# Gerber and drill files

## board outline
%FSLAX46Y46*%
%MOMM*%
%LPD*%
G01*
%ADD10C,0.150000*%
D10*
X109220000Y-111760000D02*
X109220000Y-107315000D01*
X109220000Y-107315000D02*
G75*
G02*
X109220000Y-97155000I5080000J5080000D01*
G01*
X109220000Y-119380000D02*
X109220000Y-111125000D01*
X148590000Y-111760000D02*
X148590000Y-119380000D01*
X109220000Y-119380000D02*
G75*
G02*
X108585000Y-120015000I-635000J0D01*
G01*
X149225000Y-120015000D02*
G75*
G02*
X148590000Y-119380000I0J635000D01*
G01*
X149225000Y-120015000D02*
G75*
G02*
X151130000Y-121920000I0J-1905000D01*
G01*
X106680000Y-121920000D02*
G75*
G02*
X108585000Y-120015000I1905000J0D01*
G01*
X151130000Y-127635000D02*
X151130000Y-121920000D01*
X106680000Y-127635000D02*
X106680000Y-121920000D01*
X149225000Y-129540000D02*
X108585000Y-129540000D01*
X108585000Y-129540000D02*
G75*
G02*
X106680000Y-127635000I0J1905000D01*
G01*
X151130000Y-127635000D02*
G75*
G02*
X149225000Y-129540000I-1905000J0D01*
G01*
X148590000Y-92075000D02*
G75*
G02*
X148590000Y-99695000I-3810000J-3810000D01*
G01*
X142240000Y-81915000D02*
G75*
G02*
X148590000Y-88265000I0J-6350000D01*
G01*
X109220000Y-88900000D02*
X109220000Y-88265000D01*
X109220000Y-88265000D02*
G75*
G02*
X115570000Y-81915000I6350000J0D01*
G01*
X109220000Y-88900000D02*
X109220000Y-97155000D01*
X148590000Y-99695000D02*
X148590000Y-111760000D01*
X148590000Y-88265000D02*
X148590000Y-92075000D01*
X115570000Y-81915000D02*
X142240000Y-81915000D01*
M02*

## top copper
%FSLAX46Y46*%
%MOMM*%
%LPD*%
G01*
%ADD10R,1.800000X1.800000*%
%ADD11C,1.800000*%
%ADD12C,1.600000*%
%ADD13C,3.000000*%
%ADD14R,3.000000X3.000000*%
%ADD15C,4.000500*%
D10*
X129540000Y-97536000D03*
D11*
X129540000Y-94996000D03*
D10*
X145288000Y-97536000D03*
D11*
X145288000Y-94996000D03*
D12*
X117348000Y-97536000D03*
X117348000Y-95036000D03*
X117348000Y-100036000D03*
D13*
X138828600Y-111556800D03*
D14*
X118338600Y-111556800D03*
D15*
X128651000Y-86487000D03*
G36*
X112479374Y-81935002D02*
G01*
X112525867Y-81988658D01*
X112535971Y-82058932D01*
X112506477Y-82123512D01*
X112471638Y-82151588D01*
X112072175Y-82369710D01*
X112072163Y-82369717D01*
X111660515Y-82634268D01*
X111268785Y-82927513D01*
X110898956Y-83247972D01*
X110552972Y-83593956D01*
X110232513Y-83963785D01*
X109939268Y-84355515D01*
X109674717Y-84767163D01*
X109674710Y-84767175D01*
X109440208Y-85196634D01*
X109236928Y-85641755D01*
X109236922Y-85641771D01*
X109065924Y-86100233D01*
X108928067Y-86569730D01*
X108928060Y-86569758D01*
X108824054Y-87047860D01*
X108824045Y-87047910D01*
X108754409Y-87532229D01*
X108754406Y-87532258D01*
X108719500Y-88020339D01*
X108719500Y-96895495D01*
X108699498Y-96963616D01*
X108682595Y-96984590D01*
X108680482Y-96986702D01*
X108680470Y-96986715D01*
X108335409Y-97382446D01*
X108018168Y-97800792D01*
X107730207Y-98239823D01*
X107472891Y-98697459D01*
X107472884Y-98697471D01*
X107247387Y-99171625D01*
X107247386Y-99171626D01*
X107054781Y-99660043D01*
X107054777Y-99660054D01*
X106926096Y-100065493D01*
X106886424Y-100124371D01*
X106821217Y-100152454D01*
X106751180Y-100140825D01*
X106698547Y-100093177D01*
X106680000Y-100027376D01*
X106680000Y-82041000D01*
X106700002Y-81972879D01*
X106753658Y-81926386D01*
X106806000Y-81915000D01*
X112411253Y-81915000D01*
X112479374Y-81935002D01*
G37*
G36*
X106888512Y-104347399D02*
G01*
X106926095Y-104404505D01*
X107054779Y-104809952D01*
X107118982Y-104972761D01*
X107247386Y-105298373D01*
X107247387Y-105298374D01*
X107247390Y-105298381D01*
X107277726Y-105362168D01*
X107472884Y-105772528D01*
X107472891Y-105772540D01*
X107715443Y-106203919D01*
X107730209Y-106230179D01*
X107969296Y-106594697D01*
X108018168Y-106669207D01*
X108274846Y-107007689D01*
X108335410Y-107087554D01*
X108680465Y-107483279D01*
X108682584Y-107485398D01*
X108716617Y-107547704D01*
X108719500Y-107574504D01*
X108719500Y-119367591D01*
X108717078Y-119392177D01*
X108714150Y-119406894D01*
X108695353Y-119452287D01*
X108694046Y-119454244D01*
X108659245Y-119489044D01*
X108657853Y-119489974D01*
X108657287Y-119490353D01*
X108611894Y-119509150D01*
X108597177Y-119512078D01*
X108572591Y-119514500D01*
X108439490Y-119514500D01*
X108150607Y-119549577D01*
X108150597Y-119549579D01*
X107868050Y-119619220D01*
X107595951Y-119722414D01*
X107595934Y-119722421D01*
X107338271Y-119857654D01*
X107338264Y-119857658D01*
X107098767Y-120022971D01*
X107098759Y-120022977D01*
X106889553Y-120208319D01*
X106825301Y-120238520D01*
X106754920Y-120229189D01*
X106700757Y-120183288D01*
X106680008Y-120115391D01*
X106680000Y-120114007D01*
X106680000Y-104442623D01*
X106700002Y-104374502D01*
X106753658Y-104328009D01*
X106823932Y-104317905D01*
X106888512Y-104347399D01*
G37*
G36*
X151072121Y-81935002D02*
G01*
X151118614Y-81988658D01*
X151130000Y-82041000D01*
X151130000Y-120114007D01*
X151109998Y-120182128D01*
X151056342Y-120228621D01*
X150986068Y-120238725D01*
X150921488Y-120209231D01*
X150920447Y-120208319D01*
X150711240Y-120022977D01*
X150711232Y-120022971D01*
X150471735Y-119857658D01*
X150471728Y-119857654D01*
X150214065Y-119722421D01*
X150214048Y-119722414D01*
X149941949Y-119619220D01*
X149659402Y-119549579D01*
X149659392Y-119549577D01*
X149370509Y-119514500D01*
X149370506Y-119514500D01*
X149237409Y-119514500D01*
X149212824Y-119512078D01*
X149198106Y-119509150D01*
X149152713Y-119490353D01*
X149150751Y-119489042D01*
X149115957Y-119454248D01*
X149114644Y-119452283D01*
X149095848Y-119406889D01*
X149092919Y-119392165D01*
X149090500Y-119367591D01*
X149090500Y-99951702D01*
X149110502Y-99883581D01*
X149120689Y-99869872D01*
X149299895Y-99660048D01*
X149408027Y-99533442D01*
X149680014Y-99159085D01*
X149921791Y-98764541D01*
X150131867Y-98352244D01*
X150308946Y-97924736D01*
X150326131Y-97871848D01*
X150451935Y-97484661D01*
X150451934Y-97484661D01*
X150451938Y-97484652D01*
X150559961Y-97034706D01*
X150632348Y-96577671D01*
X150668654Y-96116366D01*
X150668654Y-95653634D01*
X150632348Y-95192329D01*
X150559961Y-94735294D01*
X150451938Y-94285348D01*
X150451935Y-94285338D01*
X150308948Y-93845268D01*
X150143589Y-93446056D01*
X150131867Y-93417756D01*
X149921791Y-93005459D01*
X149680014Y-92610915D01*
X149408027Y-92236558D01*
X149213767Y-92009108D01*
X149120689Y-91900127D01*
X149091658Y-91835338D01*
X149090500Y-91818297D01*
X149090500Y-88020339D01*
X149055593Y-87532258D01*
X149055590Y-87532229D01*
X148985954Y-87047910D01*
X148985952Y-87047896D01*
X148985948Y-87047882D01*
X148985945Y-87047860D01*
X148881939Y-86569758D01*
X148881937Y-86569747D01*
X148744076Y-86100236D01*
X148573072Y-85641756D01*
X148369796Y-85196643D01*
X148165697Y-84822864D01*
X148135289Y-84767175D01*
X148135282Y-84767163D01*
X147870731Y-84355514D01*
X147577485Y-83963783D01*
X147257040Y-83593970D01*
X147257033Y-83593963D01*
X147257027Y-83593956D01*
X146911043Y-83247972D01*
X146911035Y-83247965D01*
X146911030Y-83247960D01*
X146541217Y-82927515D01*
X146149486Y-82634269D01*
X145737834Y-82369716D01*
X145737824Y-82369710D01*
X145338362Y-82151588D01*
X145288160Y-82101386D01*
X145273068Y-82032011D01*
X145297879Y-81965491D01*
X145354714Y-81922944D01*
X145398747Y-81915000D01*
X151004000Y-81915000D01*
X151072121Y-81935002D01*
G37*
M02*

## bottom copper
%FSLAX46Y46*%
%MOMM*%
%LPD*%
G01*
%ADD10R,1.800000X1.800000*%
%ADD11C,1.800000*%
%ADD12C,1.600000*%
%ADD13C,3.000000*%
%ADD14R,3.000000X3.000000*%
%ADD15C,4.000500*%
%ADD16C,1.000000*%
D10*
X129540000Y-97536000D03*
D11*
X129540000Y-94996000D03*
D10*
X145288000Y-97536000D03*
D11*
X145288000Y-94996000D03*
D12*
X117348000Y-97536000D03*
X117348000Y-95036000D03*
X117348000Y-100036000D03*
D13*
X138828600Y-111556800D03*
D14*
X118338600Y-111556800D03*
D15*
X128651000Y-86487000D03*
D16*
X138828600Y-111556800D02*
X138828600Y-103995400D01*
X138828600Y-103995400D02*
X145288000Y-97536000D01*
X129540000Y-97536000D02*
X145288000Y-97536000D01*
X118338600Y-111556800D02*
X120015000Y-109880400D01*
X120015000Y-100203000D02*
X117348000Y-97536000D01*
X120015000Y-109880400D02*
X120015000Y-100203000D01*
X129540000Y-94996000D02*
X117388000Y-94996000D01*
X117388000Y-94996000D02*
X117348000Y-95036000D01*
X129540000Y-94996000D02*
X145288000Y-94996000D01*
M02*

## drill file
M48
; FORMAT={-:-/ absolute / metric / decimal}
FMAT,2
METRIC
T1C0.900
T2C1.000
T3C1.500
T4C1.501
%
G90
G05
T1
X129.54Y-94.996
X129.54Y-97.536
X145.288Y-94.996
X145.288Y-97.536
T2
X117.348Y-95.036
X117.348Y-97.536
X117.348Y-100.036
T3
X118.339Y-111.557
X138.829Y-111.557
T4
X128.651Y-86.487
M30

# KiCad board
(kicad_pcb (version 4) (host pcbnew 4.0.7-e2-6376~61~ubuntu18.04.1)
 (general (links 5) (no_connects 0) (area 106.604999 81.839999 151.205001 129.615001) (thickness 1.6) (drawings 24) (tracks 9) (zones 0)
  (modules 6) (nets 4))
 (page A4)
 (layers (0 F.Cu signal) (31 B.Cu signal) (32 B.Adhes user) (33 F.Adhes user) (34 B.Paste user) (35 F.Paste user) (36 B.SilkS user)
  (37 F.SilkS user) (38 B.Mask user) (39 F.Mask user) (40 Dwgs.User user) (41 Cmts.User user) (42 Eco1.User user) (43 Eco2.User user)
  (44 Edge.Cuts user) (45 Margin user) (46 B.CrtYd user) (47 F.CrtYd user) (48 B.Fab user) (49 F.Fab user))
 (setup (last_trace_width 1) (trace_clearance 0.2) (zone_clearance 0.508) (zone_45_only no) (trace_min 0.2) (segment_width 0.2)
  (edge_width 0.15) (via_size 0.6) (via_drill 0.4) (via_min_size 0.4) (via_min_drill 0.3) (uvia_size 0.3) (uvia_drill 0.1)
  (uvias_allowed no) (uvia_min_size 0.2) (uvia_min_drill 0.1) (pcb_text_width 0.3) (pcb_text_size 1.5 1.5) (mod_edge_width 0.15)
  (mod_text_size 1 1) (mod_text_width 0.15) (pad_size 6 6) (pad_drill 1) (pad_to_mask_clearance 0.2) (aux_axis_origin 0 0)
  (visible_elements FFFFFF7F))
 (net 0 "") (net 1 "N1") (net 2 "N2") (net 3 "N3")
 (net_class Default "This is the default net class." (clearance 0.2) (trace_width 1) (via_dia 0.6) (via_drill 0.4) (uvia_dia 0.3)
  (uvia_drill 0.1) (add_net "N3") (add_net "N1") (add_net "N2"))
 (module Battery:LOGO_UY (layer F.Cu) (at 129.032 106.172)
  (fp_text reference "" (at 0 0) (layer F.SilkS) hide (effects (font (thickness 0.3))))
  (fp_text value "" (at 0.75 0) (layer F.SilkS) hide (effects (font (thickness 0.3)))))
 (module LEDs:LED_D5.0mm (layer B.Cu) (at 129.54 97.536 90)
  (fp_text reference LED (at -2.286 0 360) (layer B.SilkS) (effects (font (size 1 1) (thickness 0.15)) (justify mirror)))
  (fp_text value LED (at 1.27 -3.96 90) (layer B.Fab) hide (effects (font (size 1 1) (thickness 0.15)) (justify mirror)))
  (pad 1 thru_hole rect (at 0 0 90) (size 1.8 1.8) (drill 0.9) (layers *.Cu *.Mask) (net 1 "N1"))
  (pad 2 thru_hole circle (at 2.54 0 90) (size 1.8 1.8) (drill 0.9) (layers *.Cu *.Mask) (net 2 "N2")))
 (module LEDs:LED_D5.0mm (layer B.Cu) (at 145.288 97.536 90)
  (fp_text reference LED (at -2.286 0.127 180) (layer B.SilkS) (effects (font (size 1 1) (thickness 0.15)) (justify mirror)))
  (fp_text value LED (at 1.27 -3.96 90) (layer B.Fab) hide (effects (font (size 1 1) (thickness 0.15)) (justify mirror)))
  (pad 1 thru_hole rect (at 0 0 90) (size 1.8 1.8) (drill 0.9) (layers *.Cu *.Mask) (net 1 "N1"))
  (pad 2 thru_hole circle (at 2.54 0 90) (size 1.8 1.8) (drill 0.9) (layers *.Cu *.Mask) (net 2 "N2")))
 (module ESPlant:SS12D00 (layer B.Cu) (at 117.348 97.536 270)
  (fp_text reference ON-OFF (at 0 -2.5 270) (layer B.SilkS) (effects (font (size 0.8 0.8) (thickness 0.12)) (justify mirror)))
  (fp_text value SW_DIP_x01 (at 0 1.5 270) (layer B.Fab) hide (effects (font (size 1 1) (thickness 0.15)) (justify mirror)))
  (pad 2 thru_hole circle (at 0 0 270) (size 1.6 1.6) (drill 1) (layers *.Cu *.Mask B.SilkS) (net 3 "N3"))
  (pad 1 thru_hole circle (at -2.5 0 270) (size 1.6 1.6) (drill 1) (layers *.Cu *.Mask B.SilkS) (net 2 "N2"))
  (pad 3 thru_hole circle (at 2.5 0 270) (size 1.6 1.6) (drill 1) (layers *.Cu *.Mask B.SilkS)))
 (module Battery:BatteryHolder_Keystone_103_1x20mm (layer B.Cu) (at 118.3386 111.5568)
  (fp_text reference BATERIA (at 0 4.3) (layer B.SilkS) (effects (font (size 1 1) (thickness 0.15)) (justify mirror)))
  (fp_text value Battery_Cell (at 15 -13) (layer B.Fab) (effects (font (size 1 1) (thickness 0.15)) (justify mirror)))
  (pad 2 thru_hole circle (at 20.49 0) (size 3 3) (drill 1.5) (layers *.Cu *.Mask) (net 1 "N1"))
  (pad 1 thru_hole rect (at 0 0) (size 3 3) (drill 1.5) (layers *.Cu *.Mask) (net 3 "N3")))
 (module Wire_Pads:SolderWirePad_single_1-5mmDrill (layer F.Cu) (at 128.651 86.487)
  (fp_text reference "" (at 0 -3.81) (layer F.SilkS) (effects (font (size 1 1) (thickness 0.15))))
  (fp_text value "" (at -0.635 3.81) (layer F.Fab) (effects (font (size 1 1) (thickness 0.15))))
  (pad 1 thru_hole circle (at 0 0) (size 4.0005 4.0005) (drill 1.50114) (layers *.Cu *.Mask)))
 (gr_line (start 109.22 111.76) (end 109.22 107.315) (angle 90) (layer Edge.Cuts) (width 0.15))
 (gr_arc (start 114.3 102.235) (end 109.22 107.315) (angle 90) (layer Edge.Cuts) (width 0.15))
 (gr_line (start 109.22 119.38) (end 109.22 111.125) (angle 90) (layer Edge.Cuts) (width 0.15))
 (gr_line (start 148.59 111.76) (end 148.59 119.38) (angle 90) (layer Edge.Cuts) (width 0.15))
 (gr_arc (start 108.585 119.38) (end 109.22 119.38) (angle 90) (layer Edge.Cuts) (width 0.15))
 (gr_arc (start 149.225 119.38) (end 149.225 120.015) (angle 90) (layer Edge.Cuts) (width 0.15))
 (gr_arc (start 149.225 121.92) (end 149.225 120.015) (angle 90) (layer Edge.Cuts) (width 0.15))
 (gr_arc (start 108.585 121.92) (end 106.68 121.92) (angle 90) (layer Edge.Cuts) (width 0.15))
 (gr_line (start 151.13 127.635) (end 151.13 121.92) (angle 90) (layer Edge.Cuts) (width 0.15))
 (gr_line (start 106.68 127.635) (end 106.68 121.92) (angle 90) (layer Edge.Cuts) (width 0.15))
 (gr_line (start 149.225 129.54) (end 108.585 129.54) (angle 90) (layer Edge.Cuts) (width 0.15))
 (gr_arc (start 108.585 127.635) (end 108.585 129.54) (angle 90) (layer Edge.Cuts) (width 0.15))
 (gr_arc (start 149.225 127.635) (end 151.13 127.635) (angle 90) (layer Edge.Cuts) (width 0.15))
 (gr_arc (start 144.78 95.885) (end 148.59 92.075) (angle 90) (layer Edge.Cuts) (width 0.15))
 (gr_arc (start 142.24 88.265) (end 142.24 81.915) (angle 90) (layer Edge.Cuts) (width 0.15))
 (gr_line (start 109.22 88.9) (end 109.22 88.265) (angle 90) (layer Edge.Cuts) (width 0.15))
 (gr_arc (start 115.57 88.265) (end 109.22 88.265) (angle 90) (layer Edge.Cuts) (width 0.15))
 (gr_line (start 109.22 88.9) (end 109.22 97.155) (angle 90) (layer Edge.Cuts) (width 0.15))
 (gr_line (start 148.59 99.695) (end 148.59 111.76) (angle 90) (layer Edge.Cuts) (width 0.15))
 (gr_line (start 148.59 88.265) (end 148.59 92.075) (angle 90) (layer Edge.Cuts) (width 0.15))
 (gr_line (start 115.57 81.915) (end 142.24 81.915) (angle 90) (layer Edge.Cuts) (width 0.15))
 (segment (start 138.8286 111.5568) (end 138.8286 103.9954) (width 1) (layer B.Cu) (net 1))
 (segment (start 138.8286 103.9954) (end 145.288 97.536) (width 1) (layer B.Cu) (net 1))
 (segment (start 129.54 97.536) (end 145.288 97.536) (width 1) (layer B.Cu) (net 1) (status 80000))
 (segment (start 118.3386 111.5568) (end 120.015 109.8804) (width 1) (layer B.Cu) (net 3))
 (segment (start 120.015 100.203) (end 117.348 97.536) (width 1) (layer B.Cu) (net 3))
 (segment (start 120.015 109.8804) (end 120.015 100.203) (width 1) (layer B.Cu) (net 3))
 (segment (start 129.54 94.996) (end 117.388 94.996) (width 1) (layer B.Cu) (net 2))
 (segment (start 117.388 94.996) (end 117.348 95.036) (width 1) (layer B.Cu) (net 2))
 (segment (start 129.54 94.996) (end 145.288 94.996) (width 1) (layer B.Cu) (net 2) (status 80000))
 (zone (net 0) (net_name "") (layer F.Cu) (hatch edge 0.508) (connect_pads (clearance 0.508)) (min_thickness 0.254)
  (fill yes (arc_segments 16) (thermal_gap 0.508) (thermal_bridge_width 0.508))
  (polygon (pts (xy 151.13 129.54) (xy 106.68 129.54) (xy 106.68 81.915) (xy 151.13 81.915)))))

